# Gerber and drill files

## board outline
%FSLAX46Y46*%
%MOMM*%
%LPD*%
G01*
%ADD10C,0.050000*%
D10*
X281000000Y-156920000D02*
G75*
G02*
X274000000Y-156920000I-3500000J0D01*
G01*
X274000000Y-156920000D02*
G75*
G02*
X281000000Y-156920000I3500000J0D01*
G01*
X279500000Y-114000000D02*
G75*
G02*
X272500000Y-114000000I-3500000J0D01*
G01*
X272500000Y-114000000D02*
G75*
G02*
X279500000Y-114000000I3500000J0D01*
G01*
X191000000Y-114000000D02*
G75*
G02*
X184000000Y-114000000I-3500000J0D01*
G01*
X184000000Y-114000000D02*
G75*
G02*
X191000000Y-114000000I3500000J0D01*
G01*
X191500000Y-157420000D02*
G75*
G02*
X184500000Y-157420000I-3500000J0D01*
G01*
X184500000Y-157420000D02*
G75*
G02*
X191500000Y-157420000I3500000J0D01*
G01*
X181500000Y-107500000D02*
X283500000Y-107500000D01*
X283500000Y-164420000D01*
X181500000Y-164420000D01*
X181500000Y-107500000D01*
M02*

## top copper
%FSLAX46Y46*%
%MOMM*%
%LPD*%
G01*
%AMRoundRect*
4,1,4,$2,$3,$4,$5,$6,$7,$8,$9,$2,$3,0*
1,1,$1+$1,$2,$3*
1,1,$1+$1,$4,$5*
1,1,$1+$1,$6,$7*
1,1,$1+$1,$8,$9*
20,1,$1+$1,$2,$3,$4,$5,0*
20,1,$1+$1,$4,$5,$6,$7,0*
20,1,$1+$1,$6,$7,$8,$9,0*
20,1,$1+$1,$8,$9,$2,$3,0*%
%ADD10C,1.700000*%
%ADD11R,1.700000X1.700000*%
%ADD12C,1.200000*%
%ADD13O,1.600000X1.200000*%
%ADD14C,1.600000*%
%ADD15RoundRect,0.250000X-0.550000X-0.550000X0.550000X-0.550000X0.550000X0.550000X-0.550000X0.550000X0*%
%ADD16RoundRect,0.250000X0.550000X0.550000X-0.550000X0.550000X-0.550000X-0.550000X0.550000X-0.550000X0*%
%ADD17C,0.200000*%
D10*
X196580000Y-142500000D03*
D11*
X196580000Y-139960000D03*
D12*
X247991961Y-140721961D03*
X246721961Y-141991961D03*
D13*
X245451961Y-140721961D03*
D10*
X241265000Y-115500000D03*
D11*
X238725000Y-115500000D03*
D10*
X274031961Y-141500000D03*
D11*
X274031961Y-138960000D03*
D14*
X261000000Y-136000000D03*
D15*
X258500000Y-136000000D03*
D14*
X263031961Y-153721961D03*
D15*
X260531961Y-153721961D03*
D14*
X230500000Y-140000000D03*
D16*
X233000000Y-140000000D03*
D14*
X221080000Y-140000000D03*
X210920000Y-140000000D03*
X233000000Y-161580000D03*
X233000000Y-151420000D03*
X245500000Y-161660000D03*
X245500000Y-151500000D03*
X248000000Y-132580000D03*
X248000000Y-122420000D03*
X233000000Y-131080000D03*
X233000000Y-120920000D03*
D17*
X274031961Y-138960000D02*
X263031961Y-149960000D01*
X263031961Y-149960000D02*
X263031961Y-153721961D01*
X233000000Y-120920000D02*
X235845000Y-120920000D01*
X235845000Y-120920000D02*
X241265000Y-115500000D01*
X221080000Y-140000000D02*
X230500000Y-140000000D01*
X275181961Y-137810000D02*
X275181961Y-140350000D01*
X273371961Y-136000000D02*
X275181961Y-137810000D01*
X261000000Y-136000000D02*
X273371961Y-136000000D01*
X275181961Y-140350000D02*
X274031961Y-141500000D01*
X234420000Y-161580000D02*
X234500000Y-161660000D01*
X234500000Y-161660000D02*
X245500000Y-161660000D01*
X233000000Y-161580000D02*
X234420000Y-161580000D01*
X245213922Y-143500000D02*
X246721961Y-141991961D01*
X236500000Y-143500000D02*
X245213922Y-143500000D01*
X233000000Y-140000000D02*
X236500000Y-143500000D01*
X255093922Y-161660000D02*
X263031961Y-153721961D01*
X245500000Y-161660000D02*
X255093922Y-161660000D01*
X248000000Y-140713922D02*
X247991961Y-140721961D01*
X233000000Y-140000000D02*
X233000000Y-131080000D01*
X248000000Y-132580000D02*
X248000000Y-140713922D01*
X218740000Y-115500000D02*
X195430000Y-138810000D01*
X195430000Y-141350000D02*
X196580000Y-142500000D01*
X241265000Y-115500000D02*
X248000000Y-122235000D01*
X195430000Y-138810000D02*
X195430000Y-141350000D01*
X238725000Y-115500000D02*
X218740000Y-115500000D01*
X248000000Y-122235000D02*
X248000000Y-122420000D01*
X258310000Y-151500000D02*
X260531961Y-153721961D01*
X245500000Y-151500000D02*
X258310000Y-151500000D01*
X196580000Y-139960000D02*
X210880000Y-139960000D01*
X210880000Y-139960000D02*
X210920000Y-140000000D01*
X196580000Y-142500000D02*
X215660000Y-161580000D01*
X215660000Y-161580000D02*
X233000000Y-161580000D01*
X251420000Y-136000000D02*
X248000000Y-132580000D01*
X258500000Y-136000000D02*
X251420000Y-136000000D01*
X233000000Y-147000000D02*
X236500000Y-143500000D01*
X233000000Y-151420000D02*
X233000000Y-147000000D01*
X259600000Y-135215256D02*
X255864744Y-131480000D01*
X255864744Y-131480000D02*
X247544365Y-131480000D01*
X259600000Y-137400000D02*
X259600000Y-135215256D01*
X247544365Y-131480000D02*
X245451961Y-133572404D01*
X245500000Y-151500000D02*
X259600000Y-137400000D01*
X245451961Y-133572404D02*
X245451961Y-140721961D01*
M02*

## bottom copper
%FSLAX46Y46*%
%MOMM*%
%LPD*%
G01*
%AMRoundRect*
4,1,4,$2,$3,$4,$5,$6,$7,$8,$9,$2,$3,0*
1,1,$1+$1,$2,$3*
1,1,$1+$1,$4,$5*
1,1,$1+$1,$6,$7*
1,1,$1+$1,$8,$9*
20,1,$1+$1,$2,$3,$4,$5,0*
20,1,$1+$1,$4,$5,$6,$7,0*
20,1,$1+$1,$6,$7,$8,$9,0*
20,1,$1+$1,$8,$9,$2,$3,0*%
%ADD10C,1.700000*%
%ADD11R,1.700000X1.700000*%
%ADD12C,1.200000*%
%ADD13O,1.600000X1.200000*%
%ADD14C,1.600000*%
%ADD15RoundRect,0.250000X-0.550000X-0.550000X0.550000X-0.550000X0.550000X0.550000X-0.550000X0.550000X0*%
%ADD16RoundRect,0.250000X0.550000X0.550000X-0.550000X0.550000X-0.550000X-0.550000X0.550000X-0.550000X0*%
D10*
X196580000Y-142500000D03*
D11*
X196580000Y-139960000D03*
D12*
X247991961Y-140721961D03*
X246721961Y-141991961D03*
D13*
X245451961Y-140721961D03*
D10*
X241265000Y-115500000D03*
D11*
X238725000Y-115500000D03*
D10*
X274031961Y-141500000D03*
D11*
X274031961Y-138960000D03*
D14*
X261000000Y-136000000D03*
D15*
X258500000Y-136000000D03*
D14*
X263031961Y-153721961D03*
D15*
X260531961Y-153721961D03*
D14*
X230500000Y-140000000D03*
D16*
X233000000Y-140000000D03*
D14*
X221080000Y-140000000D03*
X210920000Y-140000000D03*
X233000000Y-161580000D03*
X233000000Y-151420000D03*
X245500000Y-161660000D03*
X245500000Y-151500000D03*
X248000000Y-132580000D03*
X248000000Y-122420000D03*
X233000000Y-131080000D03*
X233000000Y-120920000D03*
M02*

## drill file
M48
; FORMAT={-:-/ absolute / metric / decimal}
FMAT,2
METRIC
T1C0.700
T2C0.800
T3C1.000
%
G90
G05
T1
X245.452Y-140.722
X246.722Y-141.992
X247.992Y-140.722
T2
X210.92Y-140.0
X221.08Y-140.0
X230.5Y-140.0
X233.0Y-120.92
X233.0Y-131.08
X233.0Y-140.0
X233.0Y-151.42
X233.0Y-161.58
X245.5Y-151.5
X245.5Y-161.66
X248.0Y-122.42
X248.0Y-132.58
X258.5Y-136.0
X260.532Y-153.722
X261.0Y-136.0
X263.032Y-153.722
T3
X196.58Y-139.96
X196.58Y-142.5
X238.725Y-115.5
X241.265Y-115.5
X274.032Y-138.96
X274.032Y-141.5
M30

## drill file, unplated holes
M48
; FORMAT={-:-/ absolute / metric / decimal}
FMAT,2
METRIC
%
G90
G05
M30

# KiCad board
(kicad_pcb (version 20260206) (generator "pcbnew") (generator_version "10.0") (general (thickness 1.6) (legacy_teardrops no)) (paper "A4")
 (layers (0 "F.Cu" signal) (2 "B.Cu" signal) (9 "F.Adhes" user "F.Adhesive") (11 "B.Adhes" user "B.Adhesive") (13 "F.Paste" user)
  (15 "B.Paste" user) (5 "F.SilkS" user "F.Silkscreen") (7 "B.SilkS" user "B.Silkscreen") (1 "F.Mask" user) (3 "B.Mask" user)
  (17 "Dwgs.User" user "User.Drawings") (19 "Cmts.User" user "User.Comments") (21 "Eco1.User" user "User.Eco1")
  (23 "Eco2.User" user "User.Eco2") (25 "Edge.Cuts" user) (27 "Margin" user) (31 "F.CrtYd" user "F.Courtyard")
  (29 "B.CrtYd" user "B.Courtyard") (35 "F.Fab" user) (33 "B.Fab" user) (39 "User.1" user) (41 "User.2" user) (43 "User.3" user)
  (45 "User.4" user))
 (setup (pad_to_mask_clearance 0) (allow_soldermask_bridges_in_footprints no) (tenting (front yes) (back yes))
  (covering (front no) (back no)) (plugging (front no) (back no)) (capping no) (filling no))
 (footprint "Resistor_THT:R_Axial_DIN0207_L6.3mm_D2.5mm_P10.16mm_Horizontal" (layer "F.Cu") (at 245.5 151.5 -90)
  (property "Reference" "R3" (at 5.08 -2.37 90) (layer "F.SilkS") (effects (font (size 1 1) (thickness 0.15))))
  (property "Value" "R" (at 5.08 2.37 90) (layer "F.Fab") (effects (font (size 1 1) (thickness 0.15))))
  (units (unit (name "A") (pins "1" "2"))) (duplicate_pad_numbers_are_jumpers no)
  (pad "1" thru_hole circle (at 0 0 270) (size 1.6 1.6) (drill 0.8) (layers "*.Cu" "*.Mask") (remove_unused_layers no) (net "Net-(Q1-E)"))
  (pad "2" thru_hole circle (at 10.16 0 270) (size 1.6 1.6) (drill 0.8) (layers "*.Cu" "*.Mask") (remove_unused_layers no) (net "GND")))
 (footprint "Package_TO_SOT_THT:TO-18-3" (layer "F.Cu") (at 245.451961 140.721961)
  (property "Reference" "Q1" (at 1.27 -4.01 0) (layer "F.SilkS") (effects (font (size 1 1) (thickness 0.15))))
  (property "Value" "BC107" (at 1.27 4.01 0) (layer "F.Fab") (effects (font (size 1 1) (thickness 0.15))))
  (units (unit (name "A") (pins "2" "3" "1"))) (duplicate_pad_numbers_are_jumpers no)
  (pad "1" thru_hole oval (at 0 0) (size 1.6 1.2) (drill 0.7) (layers "*.Cu" "*.Mask") (remove_unused_layers no) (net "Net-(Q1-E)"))
  (pad "2" thru_hole circle (at 1.27 1.27) (size 1.2 1.2) (drill 0.7) (layers "*.Cu" "*.Mask") (remove_unused_layers no) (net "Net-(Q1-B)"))
  (pad "3" thru_hole circle (at 2.54 0) (size 1.2 1.2) (drill 0.7) (layers "*.Cu" "*.Mask") (remove_unused_layers no) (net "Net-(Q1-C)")))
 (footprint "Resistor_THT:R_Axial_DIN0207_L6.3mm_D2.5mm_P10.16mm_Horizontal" (layer "F.Cu") (at 210.92 140)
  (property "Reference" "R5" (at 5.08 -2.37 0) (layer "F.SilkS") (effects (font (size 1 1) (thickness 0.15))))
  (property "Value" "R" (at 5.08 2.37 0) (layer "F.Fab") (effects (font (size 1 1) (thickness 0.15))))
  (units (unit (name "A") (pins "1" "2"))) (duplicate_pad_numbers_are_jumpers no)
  (pad "1" thru_hole circle (at 0 0) (size 1.6 1.6) (drill 0.8) (layers "*.Cu" "*.Mask") (remove_unused_layers no) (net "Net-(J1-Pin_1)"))
  (pad "2" thru_hole circle (at 10.16 0) (size 1.6 1.6) (drill 0.8) (layers "*.Cu" "*.Mask") (remove_unused_layers no) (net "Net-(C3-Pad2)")))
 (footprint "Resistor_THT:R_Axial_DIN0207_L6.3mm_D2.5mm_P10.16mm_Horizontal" (layer "F.Cu") (at 248 122.42 -90)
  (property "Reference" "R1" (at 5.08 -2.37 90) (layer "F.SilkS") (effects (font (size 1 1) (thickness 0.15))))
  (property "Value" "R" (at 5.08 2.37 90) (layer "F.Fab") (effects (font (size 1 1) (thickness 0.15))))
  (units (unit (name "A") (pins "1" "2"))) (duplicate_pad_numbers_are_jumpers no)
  (pad "1" thru_hole circle (at 0 0 270) (size 1.6 1.6) (drill 0.8) (layers "*.Cu" "*.Mask") (remove_unused_layers no)
   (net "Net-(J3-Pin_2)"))
  (pad "2" thru_hole circle (at 10.16 0 270) (size 1.6 1.6) (drill 0.8) (layers "*.Cu" "*.Mask") (remove_unused_layers no)
   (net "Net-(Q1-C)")))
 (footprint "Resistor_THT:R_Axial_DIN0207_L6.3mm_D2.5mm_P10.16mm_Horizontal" (layer "F.Cu") (at 233 120.92 -90)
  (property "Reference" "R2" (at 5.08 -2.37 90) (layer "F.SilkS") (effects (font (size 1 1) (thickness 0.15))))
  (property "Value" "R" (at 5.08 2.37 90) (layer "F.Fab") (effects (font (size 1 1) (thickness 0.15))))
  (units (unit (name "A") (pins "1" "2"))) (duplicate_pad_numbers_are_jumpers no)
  (pad "1" thru_hole circle (at 0 0 270) (size 1.6 1.6) (drill 0.8) (layers "*.Cu" "*.Mask") (remove_unused_layers no)
   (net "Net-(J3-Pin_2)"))
  (pad "2" thru_hole circle (at 10.16 0 270) (size 1.6 1.6) (drill 0.8) (layers "*.Cu" "*.Mask") (remove_unused_layers no)
   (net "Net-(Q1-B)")))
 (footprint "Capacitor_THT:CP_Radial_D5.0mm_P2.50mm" (layer "F.Cu") (at 258.5 136)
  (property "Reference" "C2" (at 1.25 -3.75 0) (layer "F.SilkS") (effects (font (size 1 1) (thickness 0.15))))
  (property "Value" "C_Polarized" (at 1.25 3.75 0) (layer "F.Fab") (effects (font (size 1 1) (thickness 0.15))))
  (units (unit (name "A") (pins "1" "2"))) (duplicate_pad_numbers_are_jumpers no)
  (pad "1" thru_hole roundrect (at 0 0) (size 1.6 1.6) (drill 0.8) (layers "*.Cu" "*.Mask") (remove_unused_layers no)
   (roundrect_rratio 0.15625) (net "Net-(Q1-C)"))
  (pad "2" thru_hole circle (at 2.5 0) (size 1.6 1.6) (drill 0.8) (layers "*.Cu" "*.Mask") (remove_unused_layers no) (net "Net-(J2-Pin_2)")))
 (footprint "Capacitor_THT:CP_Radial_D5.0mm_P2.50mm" (layer "F.Cu") (at 233 140 180)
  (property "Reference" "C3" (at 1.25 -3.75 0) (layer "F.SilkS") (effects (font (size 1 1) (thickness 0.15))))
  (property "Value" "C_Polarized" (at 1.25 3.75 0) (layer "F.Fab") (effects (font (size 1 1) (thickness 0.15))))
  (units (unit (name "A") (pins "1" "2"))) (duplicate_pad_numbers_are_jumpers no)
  (pad "1" thru_hole roundrect (at 0 0 180) (size 1.6 1.6) (drill 0.8) (layers "*.Cu" "*.Mask") (remove_unused_layers no)
   (roundrect_rratio 0.15625) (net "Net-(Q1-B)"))
  (pad "2" thru_hole circle (at 2.5 0 180) (size 1.6 1.6) (drill 0.8) (layers "*.Cu" "*.Mask") (remove_unused_layers no)
   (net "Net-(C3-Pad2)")))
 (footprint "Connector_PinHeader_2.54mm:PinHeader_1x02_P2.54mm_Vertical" (layer "F.Cu") (at 238.725 115.5 90)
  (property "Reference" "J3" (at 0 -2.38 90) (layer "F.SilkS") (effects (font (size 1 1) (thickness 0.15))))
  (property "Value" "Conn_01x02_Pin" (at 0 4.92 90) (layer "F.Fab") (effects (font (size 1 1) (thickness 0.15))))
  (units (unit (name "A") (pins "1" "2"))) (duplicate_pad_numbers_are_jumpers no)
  (pad "1" thru_hole rect (at 0 0 90) (size 1.7 1.7) (drill 1) (layers "*.Cu" "*.Mask") (remove_unused_layers no) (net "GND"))
  (pad "2" thru_hole circle (at 0 2.54 90) (size 1.7 1.7) (drill 1) (layers "*.Cu" "*.Mask") (remove_unused_layers no)
   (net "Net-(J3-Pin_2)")))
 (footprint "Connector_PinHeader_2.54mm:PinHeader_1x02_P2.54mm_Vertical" (layer "F.Cu") (at 196.58 139.96)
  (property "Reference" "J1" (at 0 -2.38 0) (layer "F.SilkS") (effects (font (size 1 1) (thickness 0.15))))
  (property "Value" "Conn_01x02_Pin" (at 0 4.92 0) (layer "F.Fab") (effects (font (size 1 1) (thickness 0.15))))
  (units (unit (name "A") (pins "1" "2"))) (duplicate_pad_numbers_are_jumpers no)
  (pad "1" thru_hole rect (at 0 0) (size 1.7 1.7) (drill 1) (layers "*.Cu" "*.Mask") (remove_unused_layers no) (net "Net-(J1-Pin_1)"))
  (pad "2" thru_hole circle (at 0 2.54) (size 1.7 1.7) (drill 1) (layers "*.Cu" "*.Mask") (remove_unused_layers no) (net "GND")))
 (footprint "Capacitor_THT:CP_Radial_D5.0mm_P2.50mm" (layer "F.Cu") (at 260.531961 153.721961)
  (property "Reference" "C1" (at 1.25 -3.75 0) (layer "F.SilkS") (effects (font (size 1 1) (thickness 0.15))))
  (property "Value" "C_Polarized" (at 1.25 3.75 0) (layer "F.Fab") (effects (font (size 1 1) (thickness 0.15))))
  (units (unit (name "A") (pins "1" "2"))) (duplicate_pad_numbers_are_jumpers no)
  (pad "1" thru_hole roundrect (at 0 0) (size 1.6 1.6) (drill 0.8) (layers "*.Cu" "*.Mask") (remove_unused_layers no)
   (roundrect_rratio 0.15625) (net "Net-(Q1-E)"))
  (pad "2" thru_hole circle (at 2.5 0) (size 1.6 1.6) (drill 0.8) (layers "*.Cu" "*.Mask") (remove_unused_layers no) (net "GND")))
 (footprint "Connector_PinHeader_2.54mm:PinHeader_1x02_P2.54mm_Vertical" (layer "F.Cu") (at 274.031961 138.96)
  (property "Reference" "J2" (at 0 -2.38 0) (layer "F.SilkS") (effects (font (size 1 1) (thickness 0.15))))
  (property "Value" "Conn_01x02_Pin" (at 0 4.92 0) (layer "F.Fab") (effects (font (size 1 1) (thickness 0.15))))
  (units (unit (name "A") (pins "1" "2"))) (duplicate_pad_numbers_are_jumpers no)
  (pad "1" thru_hole rect (at 0 0) (size 1.7 1.7) (drill 1) (layers "*.Cu" "*.Mask") (remove_unused_layers no) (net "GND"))
  (pad "2" thru_hole circle (at 0 2.54) (size 1.7 1.7) (drill 1) (layers "*.Cu" "*.Mask") (remove_unused_layers no) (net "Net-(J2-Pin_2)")))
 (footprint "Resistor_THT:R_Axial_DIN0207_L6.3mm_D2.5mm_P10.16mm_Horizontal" (layer "F.Cu") (at 233 151.42 -90)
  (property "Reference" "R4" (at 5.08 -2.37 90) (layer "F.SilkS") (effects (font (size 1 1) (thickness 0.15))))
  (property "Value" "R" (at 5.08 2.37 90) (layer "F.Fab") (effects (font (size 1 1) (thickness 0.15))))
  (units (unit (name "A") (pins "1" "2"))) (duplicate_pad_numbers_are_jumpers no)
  (pad "1" thru_hole circle (at 0 0 270) (size 1.6 1.6) (drill 0.8) (layers "*.Cu" "*.Mask") (remove_unused_layers no) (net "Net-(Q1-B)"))
  (pad "2" thru_hole circle (at 10.16 0 270) (size 1.6 1.6) (drill 0.8) (layers "*.Cu" "*.Mask") (remove_unused_layers no) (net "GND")))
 (gr_rect (start 181.5 107.5) (end 283.5 164.42) (stroke (width 0.05) (type default)) (fill no) (layer "Edge.Cuts"))
 (gr_circle (center 187.5 114) (end 191 114) (stroke (width 0.05) (type solid)) (fill no) (layer "Edge.Cuts"))
 (gr_circle (center 188 157.42) (end 191.5 157.42) (stroke (width 0.05) (type solid)) (fill no) (layer "Edge.Cuts"))
 (gr_circle (center 276 114) (end 279.5 114) (stroke (width 0.05) (type solid)) (fill no) (layer "Edge.Cuts"))
 (gr_circle (center 277.5 156.92) (end 281 156.92) (stroke (width 0.05) (type solid)) (fill no) (layer "Edge.Cuts"))
 (segment (start 255.864744 131.48) (end 247.544365 131.48) (width 0.2) (layer "F.Cu") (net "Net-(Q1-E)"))
 (segment (start 259.6 135.215256) (end 255.864744 131.48) (width 0.2) (layer "F.Cu") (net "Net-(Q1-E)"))
 (segment (start 245.5 151.5) (end 259.6 137.4) (width 0.2) (layer "F.Cu") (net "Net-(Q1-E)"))
 (segment (start 258.31 151.5) (end 260.531961 153.721961) (width 0.2) (layer "F.Cu") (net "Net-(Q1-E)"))
 (segment (start 247.544365 131.48) (end 245.451961 133.572404) (width 0.2) (layer "F.Cu") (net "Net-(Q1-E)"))
 (segment (start 245.5 151.5) (end 258.31 151.5) (width 0.2) (layer "F.Cu") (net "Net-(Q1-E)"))
 (segment (start 259.6 137.4) (end 259.6 135.215256) (width 0.2) (layer "F.Cu") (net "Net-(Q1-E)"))
 (segment (start 245.451961 133.572404) (end 245.451961 140.721961) (width 0.2) (layer "F.Cu") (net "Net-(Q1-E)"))
 (segment (start 245.5 161.66) (end 255.093922 161.66) (width 0.2) (layer "F.Cu") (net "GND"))
 (segment (start 233 161.58) (end 234.42 161.58) (width 0.2) (layer "F.Cu") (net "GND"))
 (segment (start 234.5 161.66) (end 245.5 161.66) (width 0.2) (layer "F.Cu") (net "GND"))
 (segment (start 195.43 138.81) (end 195.43 141.35) (width 0.2) (layer "F.Cu") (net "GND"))
 (segment (start 255.093922 161.66) (end 263.031961 153.721961) (width 0.2) (layer "F.Cu") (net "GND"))
 (segment (start 238.725 115.5) (end 218.74 115.5) (width 0.2) (layer "F.Cu") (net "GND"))
 (segment (start 234.42 161.58) (end 234.5 161.66) (width 0.2) (layer "F.Cu") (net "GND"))
 (segment (start 274.031961 138.96) (end 263.031961 149.96) (width 0.2) (layer "F.Cu") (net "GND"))
 (segment (start 196.58 142.5) (end 215.66 161.58) (width 0.2) (layer "F.Cu") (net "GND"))
 (segment (start 218.74 115.5) (end 195.43 138.81) (width 0.2) (layer "F.Cu") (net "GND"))
 (segment (start 195.43 141.35) (end 196.58 142.5) (width 0.2) (layer "F.Cu") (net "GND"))
 (segment (start 263.031961 149.96) (end 263.031961 153.721961) (width 0.2) (layer "F.Cu") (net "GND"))
 (segment (start 215.66 161.58) (end 233 161.58) (width 0.2) (layer "F.Cu") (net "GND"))
 (segment (start 245.213922 143.5) (end 246.721961 141.991961) (width 0.2) (layer "F.Cu") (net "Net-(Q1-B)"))
 (segment (start 236.5 143.5) (end 245.213922 143.5) (width 0.2) (layer "F.Cu") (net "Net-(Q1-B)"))
 (segment (start 233 140) (end 236.5 143.5) (width 0.2) (layer "F.Cu") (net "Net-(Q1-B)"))
 (segment (start 233 151.42) (end 233 147) (width 0.2) (layer "F.Cu") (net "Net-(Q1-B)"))
 (segment (start 233 147) (end 236.5 143.5) (width 0.2) (layer "F.Cu") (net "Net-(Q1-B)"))
 (segment (start 233 140) (end 233 131.08) (width 0.2) (layer "F.Cu") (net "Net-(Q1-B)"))
 (segment (start 251.42 136) (end 248 132.58) (width 0.2) (layer "F.Cu") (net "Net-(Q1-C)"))
 (segment (start 248 140.713922) (end 247.991961 140.721961) (width 0.2) (layer "F.Cu") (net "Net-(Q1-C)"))
 (segment (start 258.5 136) (end 251.42 136) (width 0.2) (layer "F.Cu") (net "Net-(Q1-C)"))
 (segment (start 248 132.58) (end 248 140.713922) (width 0.2) (layer "F.Cu") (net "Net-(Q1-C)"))
 (segment (start 210.88 139.96) (end 210.92 140) (width 0.2) (layer "F.Cu") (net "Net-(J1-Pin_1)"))
 (segment (start 196.58 139.96) (end 210.88 139.96) (width 0.2) (layer "F.Cu") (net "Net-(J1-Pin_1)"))
 (segment (start 221.08 140) (end 230.5 140) (width 0.2) (layer "F.Cu") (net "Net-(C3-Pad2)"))
 (segment (start 235.845 120.92) (end 241.265 115.5) (width 0.2) (layer "F.Cu") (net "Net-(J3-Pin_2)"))
 (segment (start 241.265 115.5) (end 248 122.235) (width 0.2) (layer "F.Cu") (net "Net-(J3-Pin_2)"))
 (segment (start 233 120.92) (end 235.845 120.92) (width 0.2) (layer "F.Cu") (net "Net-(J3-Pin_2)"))
 (segment (start 248 122.235) (end 248 122.42) (width 0.2) (layer "F.Cu") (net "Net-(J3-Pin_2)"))
 (segment (start 261 136) (end 273.371961 136) (width 0.2) (layer "F.Cu") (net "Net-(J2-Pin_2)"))
 (segment (start 275.181961 140.35) (end 274.031961 141.5) (width 0.2) (layer "F.Cu") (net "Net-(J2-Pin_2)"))
 (segment (start 275.181961 137.81) (end 275.181961 140.35) (width 0.2) (layer "F.Cu") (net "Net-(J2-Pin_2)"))
 (segment (start 273.371961 136) (end 275.181961 137.81) (width 0.2) (layer "F.Cu") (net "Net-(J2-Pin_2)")))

